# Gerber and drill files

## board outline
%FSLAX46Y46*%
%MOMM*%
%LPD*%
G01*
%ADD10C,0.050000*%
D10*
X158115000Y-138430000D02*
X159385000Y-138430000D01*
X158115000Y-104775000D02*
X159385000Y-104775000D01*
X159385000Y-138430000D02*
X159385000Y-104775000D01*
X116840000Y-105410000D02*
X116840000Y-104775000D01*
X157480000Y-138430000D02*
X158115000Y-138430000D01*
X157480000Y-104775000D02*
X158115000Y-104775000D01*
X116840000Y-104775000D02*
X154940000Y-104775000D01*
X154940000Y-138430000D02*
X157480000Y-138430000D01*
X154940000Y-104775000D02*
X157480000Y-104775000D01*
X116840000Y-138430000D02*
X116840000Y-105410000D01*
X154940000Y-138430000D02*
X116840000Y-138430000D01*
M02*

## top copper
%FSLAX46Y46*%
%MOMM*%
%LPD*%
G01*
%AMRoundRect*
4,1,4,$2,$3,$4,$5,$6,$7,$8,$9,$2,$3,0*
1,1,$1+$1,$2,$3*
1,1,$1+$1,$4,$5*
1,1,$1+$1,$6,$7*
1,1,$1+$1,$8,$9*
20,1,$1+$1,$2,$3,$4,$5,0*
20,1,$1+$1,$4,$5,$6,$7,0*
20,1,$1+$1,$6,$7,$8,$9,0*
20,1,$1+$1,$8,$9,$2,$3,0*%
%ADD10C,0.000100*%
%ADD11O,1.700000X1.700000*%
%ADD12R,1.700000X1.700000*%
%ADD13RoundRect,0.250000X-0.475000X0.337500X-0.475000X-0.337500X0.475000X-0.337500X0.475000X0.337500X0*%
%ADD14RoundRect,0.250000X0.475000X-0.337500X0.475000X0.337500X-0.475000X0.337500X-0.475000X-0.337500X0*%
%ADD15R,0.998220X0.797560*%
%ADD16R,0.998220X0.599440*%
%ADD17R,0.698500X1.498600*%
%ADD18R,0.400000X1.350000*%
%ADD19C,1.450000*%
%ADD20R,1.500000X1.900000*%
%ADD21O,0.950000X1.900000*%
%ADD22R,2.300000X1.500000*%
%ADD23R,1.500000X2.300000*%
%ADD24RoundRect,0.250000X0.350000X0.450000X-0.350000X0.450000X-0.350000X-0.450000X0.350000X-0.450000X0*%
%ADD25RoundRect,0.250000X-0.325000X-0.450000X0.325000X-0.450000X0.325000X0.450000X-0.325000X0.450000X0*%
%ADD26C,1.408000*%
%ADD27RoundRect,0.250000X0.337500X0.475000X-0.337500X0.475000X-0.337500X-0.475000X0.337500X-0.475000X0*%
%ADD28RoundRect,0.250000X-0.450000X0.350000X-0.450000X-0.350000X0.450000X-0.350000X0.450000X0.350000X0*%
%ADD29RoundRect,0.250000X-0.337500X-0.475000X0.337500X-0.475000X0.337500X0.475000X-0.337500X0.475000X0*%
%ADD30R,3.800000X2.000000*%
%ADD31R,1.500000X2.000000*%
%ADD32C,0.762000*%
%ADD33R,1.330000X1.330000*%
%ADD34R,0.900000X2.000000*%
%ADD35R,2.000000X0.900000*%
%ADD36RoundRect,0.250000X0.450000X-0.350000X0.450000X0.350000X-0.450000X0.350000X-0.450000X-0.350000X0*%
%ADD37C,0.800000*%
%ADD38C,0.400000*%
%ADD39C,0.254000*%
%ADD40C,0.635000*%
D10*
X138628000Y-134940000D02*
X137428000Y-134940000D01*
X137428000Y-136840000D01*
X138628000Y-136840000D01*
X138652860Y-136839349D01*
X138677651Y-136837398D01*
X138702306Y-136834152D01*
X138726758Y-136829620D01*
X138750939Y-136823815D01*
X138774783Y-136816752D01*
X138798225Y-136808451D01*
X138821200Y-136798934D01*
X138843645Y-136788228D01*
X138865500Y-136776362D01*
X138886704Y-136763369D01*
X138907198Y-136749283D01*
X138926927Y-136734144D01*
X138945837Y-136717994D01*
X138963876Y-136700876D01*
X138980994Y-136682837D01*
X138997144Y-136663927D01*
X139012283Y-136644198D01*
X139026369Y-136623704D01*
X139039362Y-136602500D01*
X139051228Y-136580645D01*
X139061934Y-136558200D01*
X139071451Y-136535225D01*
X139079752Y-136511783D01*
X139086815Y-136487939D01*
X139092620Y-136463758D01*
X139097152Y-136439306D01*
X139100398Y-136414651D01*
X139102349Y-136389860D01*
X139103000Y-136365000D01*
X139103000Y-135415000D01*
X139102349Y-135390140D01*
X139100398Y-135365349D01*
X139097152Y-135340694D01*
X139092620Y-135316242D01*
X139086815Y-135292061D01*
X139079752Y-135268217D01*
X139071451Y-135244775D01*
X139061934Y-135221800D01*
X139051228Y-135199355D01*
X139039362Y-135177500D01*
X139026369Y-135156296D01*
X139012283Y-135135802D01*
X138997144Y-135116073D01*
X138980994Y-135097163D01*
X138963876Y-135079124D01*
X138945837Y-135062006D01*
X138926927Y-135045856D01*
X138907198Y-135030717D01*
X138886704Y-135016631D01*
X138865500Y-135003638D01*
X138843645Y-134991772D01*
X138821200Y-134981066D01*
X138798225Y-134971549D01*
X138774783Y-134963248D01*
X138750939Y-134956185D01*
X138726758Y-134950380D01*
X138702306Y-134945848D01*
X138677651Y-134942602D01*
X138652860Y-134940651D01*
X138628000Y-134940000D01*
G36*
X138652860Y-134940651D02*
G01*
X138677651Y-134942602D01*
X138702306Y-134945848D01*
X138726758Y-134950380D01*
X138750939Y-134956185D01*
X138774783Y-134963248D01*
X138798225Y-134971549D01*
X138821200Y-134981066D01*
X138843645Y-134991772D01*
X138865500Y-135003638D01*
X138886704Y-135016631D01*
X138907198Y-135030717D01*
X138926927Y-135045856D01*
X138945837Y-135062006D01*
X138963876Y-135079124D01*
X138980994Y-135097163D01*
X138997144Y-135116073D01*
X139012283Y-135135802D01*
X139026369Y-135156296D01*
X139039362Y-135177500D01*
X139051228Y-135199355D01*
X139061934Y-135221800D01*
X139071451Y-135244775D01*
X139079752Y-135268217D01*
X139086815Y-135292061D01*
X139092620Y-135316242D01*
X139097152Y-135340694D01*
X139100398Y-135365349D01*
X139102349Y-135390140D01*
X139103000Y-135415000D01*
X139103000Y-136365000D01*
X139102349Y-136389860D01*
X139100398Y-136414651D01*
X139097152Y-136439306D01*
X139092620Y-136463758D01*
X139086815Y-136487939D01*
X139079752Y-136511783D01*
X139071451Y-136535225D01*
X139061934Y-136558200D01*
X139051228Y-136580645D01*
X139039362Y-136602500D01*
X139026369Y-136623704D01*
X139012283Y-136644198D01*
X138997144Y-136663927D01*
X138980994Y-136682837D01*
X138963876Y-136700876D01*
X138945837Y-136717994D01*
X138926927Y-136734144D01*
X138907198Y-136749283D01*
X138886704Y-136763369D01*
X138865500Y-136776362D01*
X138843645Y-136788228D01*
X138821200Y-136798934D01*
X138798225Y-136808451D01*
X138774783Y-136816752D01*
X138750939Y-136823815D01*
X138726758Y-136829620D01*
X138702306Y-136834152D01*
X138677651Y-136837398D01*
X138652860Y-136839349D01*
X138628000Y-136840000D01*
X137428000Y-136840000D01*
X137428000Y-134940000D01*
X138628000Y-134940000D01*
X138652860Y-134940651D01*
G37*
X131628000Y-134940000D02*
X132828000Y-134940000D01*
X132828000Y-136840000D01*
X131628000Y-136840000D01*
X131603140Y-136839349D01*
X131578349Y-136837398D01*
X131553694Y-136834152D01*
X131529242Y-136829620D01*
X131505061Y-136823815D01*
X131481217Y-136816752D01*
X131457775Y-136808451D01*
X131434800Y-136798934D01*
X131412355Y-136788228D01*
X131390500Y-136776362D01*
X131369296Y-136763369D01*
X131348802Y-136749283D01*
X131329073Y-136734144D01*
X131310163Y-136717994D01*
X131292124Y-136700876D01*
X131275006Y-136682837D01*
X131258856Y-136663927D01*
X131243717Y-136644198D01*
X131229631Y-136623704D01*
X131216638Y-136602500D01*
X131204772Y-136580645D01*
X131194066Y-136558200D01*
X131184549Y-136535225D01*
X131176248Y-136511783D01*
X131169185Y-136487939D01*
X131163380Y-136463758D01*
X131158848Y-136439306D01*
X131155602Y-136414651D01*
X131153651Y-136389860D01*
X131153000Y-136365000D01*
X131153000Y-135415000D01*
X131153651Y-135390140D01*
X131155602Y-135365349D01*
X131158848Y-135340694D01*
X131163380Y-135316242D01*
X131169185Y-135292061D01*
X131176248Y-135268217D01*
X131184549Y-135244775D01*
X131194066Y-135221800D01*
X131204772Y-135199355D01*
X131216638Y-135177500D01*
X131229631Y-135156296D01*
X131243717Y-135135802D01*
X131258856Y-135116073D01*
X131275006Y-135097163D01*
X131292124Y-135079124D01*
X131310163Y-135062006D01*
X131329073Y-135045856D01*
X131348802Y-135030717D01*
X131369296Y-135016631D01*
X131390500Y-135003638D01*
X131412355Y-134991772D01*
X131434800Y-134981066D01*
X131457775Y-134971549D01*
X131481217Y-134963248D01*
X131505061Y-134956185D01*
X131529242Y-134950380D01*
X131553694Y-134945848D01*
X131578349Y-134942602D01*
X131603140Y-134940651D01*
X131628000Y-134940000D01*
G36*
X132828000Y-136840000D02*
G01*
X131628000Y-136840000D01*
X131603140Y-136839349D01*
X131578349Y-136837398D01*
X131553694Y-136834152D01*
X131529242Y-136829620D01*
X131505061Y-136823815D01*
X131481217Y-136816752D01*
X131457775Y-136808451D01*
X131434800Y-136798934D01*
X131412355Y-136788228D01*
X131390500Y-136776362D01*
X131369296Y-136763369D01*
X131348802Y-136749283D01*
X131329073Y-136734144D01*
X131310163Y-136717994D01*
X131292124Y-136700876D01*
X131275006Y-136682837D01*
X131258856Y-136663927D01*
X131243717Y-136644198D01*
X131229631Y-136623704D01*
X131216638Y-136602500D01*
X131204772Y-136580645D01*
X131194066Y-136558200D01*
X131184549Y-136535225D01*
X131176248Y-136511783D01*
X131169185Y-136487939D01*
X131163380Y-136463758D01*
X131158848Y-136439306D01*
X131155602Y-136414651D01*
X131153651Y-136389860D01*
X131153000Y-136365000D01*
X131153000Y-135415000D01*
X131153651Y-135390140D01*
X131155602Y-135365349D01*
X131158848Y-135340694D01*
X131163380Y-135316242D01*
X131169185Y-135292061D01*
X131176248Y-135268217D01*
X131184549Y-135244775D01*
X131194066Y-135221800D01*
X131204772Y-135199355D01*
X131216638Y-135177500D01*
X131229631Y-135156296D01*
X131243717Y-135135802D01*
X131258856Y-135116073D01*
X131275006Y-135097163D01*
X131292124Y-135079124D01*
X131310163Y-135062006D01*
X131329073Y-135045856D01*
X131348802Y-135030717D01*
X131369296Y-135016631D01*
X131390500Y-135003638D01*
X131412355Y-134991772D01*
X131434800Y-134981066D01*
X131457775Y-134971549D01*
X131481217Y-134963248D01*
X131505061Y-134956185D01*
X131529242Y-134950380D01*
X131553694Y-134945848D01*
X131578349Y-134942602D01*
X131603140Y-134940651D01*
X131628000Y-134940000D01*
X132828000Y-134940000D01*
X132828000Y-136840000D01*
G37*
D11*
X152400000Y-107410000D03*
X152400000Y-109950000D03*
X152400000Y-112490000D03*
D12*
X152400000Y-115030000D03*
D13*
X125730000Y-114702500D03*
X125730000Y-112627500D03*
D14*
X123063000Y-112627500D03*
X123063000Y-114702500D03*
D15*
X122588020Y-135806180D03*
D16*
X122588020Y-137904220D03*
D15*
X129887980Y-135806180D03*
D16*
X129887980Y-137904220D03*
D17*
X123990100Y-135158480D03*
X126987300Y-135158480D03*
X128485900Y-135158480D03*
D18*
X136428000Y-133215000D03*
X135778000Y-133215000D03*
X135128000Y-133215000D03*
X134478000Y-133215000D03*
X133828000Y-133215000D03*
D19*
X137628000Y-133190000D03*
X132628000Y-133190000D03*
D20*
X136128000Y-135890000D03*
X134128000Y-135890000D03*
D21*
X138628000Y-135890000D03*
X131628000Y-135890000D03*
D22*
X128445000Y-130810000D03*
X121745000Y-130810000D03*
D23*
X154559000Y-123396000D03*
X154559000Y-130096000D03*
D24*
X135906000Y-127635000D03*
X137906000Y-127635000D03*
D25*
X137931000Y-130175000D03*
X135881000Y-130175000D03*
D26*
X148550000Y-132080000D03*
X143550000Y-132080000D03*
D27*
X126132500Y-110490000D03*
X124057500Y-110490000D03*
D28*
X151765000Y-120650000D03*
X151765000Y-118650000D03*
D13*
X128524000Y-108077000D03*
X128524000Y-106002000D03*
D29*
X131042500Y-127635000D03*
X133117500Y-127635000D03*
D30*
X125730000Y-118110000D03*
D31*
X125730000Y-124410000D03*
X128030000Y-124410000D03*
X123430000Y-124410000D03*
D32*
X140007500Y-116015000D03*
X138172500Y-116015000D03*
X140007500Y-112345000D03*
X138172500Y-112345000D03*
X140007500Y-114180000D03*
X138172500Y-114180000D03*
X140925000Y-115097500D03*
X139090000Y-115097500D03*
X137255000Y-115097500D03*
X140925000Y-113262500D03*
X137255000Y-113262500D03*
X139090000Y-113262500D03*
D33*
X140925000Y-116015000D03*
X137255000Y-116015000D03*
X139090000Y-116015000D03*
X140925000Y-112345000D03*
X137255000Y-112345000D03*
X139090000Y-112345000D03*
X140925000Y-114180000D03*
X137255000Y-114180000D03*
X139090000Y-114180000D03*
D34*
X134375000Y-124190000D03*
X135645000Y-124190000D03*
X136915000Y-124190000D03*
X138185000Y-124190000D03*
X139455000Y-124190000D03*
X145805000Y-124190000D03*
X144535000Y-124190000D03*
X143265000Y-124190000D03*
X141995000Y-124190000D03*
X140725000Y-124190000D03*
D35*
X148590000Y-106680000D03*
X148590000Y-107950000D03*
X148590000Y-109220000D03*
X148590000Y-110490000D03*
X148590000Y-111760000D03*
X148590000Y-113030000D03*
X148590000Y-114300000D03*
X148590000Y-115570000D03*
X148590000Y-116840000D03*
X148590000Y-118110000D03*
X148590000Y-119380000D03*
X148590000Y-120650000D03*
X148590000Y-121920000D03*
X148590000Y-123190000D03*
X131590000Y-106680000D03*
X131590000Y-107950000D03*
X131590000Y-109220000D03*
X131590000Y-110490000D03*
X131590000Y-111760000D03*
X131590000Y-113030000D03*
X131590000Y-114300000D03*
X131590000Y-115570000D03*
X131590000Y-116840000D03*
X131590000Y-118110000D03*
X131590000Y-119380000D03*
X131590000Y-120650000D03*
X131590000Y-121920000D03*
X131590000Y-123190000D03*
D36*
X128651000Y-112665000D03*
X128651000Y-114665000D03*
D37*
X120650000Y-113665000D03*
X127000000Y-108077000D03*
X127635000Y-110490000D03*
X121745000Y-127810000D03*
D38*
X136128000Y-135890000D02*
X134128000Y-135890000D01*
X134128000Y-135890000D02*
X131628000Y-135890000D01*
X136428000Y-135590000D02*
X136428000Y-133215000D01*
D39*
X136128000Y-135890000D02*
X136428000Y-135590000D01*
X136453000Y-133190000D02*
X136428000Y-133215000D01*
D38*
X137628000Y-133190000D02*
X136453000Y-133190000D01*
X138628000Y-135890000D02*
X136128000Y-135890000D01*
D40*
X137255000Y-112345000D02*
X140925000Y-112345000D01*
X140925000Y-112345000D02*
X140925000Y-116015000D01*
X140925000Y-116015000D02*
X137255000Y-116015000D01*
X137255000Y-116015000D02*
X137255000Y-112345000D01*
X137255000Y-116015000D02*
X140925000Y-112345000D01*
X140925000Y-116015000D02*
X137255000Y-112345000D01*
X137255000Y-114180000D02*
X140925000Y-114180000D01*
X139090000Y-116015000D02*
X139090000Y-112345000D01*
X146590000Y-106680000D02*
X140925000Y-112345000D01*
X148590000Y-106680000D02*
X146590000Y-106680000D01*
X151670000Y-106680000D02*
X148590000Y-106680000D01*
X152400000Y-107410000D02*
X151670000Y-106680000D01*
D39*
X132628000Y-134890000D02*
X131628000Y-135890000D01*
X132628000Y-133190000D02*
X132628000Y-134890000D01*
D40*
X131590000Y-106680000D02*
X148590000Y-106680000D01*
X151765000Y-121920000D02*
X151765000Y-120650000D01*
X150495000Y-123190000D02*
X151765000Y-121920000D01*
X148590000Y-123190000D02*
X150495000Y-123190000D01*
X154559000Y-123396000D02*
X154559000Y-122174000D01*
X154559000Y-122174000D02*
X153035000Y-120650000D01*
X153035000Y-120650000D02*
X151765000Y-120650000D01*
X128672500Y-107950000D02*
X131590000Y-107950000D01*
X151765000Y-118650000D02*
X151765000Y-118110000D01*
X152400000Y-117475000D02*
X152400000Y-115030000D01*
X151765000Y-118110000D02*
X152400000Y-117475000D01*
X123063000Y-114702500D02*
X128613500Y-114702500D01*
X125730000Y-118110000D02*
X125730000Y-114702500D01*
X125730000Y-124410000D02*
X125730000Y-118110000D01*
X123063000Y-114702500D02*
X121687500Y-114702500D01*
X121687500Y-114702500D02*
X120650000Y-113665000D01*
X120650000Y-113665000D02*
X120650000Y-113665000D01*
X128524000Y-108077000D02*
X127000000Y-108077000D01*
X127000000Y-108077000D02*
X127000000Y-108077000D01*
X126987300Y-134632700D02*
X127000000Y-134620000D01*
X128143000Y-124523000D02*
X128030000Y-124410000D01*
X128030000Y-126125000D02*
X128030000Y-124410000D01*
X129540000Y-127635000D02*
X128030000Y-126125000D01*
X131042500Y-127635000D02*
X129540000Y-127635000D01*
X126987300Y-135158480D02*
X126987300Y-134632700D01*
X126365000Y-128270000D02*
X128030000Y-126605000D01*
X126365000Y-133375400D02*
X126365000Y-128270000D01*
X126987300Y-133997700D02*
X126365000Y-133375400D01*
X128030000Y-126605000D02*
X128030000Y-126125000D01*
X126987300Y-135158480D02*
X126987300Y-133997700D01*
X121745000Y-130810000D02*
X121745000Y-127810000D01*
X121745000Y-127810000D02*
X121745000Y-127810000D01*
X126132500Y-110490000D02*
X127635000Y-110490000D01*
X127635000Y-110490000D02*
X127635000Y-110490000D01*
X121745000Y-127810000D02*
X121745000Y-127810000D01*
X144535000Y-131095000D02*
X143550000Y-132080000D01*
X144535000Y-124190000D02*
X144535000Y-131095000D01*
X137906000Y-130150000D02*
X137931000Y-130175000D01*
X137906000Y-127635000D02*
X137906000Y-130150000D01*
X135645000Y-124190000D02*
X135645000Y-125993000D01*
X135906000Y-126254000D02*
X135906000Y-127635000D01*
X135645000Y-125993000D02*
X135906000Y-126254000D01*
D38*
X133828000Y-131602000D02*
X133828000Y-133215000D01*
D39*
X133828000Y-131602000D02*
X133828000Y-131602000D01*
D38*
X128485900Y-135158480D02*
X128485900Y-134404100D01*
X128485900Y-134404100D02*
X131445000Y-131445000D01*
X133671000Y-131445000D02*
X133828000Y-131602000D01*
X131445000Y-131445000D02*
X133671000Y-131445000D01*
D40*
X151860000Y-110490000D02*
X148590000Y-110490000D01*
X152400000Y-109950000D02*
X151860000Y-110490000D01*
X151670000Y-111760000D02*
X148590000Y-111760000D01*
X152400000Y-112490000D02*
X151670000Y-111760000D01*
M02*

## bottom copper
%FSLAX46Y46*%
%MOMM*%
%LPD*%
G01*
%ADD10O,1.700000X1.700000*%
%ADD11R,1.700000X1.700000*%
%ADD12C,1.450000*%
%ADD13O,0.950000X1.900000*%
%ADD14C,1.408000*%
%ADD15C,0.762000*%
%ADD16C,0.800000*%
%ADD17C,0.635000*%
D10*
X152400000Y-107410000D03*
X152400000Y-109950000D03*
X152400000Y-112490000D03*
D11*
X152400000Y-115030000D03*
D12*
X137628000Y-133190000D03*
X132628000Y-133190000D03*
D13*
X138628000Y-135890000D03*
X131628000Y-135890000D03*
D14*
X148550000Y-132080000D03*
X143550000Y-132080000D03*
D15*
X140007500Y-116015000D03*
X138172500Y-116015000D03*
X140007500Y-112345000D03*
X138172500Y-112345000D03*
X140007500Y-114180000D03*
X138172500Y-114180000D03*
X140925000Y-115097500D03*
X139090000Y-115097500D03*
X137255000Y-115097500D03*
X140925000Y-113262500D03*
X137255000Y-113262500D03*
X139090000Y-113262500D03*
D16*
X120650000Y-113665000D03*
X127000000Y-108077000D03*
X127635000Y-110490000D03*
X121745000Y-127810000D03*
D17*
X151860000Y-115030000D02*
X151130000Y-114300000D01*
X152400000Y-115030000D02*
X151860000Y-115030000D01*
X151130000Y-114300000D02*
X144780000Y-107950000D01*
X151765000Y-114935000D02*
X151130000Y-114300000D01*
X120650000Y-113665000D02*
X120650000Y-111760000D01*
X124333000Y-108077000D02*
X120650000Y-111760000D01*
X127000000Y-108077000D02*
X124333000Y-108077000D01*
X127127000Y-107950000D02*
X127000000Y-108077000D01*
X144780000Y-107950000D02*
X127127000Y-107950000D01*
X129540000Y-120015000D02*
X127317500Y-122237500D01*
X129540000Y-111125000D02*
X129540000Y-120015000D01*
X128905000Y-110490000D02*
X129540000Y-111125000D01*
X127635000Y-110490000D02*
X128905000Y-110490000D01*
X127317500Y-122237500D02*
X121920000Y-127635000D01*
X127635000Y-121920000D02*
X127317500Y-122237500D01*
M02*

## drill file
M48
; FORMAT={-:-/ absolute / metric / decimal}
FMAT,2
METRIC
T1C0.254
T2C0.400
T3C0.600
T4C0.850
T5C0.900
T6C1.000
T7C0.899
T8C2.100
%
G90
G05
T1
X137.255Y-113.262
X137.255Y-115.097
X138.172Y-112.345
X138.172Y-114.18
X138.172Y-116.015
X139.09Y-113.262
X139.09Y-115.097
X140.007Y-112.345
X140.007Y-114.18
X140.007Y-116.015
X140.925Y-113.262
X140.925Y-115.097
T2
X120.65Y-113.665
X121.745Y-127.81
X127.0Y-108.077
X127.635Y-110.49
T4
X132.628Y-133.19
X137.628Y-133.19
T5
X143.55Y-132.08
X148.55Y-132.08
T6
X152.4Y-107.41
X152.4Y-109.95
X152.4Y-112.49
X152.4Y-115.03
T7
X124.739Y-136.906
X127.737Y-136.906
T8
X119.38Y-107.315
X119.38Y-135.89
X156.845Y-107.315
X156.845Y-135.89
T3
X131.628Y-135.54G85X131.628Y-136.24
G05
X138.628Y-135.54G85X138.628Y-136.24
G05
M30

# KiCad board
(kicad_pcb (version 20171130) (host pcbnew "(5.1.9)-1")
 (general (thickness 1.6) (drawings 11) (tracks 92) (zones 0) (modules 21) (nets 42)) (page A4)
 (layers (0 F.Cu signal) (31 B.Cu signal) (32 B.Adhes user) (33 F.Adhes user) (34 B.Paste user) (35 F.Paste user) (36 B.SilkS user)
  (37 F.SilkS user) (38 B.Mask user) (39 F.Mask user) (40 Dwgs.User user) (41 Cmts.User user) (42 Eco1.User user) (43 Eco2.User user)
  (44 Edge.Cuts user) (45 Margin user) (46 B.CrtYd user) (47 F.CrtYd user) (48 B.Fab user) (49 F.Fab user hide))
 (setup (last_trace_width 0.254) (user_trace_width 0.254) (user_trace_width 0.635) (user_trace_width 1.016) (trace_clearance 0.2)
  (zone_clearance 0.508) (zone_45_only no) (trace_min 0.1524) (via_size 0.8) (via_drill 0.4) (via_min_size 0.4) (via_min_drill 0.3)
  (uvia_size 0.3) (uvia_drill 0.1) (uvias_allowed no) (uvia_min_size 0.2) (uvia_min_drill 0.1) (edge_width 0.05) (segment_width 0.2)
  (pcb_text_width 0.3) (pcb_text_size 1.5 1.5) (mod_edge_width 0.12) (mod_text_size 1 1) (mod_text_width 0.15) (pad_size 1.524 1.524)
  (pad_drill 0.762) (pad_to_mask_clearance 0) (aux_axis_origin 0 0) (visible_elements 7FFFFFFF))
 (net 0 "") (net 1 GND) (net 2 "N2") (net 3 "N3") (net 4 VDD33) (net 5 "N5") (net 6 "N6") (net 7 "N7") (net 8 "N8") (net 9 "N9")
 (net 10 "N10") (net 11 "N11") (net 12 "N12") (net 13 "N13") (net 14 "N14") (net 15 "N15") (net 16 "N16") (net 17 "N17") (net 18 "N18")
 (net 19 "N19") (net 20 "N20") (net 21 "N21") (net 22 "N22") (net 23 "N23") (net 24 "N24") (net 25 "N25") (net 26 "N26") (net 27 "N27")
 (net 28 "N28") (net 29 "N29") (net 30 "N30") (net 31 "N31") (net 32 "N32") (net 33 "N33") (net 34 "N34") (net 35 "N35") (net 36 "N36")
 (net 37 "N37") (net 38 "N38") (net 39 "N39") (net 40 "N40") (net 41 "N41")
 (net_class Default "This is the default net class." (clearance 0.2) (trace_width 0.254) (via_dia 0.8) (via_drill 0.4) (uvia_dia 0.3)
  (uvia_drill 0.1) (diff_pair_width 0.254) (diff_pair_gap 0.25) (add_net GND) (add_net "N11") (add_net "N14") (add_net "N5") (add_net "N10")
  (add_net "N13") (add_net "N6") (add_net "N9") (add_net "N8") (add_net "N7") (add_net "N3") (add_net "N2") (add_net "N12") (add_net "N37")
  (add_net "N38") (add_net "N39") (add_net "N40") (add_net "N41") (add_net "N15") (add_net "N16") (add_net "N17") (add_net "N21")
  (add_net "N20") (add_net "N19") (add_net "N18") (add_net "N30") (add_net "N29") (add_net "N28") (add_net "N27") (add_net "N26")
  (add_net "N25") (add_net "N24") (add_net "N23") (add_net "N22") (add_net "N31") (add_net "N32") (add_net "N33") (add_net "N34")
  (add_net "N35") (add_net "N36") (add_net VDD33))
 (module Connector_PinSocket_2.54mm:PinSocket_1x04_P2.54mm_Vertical (layer F.Cu) (at 152.4 115.03 180)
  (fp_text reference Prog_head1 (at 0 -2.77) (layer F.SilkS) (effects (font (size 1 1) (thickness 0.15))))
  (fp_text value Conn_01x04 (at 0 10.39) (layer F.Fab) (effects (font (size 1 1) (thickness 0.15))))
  (pad 4 thru_hole oval (at 0 7.62 180) (size 1.7 1.7) (drill 1) (layers *.Cu *.Mask) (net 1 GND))
  (pad 3 thru_hole oval (at 0 5.08 180) (size 1.7 1.7) (drill 1) (layers *.Cu *.Mask) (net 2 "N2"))
  (pad 2 thru_hole oval (at 0 2.54 180) (size 1.7 1.7) (drill 1) (layers *.Cu *.Mask) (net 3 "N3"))
  (pad 1 thru_hole rect (at 0 0 180) (size 1.7 1.7) (drill 1) (layers *.Cu *.Mask) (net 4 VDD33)))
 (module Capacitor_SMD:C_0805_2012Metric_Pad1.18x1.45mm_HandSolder (layer F.Cu) (at 125.73 113.665 270)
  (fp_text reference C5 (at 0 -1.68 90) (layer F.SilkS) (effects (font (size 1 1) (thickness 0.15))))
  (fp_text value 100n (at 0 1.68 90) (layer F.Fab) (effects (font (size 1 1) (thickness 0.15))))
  (pad 2 smd roundrect (at 1.0375 0 270) (size 1.175 1.45) (layers F.Cu F.Paste F.Mask) (roundrect_rratio 0.212766) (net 4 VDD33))
  (pad 1 smd roundrect (at -1.0375 0 270) (size 1.175 1.45) (layers F.Cu F.Paste F.Mask) (roundrect_rratio 0.212766) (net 1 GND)))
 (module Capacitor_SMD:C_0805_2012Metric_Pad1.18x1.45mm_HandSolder (layer F.Cu) (at 123.063 113.665 90)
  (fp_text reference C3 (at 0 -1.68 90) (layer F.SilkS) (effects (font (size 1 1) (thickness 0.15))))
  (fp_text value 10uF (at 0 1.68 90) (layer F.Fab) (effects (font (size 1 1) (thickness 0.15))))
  (pad 2 smd roundrect (at 1.0375 0 90) (size 1.175 1.45) (layers F.Cu F.Paste F.Mask) (roundrect_rratio 0.212766) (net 1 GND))
  (pad 1 smd roundrect (at -1.0375 0 90) (size 1.175 1.45) (layers F.Cu F.Paste F.Mask) (roundrect_rratio 0.212766) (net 4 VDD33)))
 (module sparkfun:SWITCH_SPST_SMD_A (layer F.Cu) (at 126.238 136.906 180)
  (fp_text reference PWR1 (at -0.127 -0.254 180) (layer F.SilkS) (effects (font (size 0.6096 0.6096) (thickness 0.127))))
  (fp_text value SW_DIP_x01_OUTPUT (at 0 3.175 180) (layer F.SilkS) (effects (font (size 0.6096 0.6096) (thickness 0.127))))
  (pad "" np_thru_hole circle (at 1.4986 0 180) (size 0.89916 0.89916) (drill 0.89916) (layers *.Cu *.Mask) (solder_mask_margin 0.1016))
  (pad "" np_thru_hole circle (at -1.4986 0 180) (size 0.89916 0.89916) (drill 0.89916) (layers *.Cu *.Mask) (solder_mask_margin 0.1016))
  (pad GND4 smd rect (at 3.64998 1.09982 180) (size 0.99822 0.79756) (layers F.Cu F.Paste F.Mask) (solder_mask_margin 0.1016))
  (pad GND3 smd rect (at 3.64998 -0.99822 180) (size 0.99822 0.59944) (layers F.Cu F.Paste F.Mask) (solder_mask_margin 0.1016))
  (pad GND2 smd rect (at -3.64998 1.09982 180) (size 0.99822 0.79756) (layers F.Cu F.Paste F.Mask) (solder_mask_margin 0.1016))
  (pad GND1 smd rect (at -3.64998 -0.99822 180) (size 0.99822 0.59944) (layers F.Cu F.Paste F.Mask) (solder_mask_margin 0.1016))
  (pad 3 smd rect (at 2.2479 1.74752) (size 0.6985 1.4986) (layers F.Cu F.Paste F.Mask) (solder_mask_margin 0.1016))
  (pad 2 smd rect (at -0.7493 1.74752) (size 0.6985 1.4986) (layers F.Cu F.Paste F.Mask) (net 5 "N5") (solder_mask_margin 0.1016))
  (pad 1 smd rect (at -2.2479 1.74752) (size 0.6985 1.4986) (layers F.Cu F.Paste F.Mask) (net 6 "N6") (solder_mask_margin 0.1016)))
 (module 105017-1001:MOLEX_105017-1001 (layer F.Cu) (at 135.128 135.89)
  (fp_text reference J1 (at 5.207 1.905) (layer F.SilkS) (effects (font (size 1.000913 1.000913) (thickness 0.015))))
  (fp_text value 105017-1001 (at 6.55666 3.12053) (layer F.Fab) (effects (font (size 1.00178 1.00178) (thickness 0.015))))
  (fp_poly
   (pts (xy 3.5 -0.95) (xy 2.3 -0.95) (xy 2.3 0.95) (xy 3.5 0.95) (xy 3.52486 0.949349) (xy 3.549651 0.947398) (xy 3.574306 0.944152)
    (xy 3.598758 0.93962) (xy 3.622939 0.933815) (xy 3.646783 0.926752) (xy 3.670225 0.918451) (xy 3.6932 0.908934) (xy 3.715645 0.898228)
    (xy 3.7375 0.886362) (xy 3.758704 0.873369) (xy 3.779198 0.859283) (xy 3.798927 0.844144) (xy 3.817837 0.827994) (xy 3.835876 0.810876)
    (xy 3.852994 0.792837) (xy 3.869144 0.773927) (xy 3.884283 0.754198) (xy 3.898369 0.733704) (xy 3.911362 0.7125) (xy 3.923228 0.690645)
    (xy 3.933934 0.6682) (xy 3.943451 0.645225) (xy 3.951752 0.621783) (xy 3.958815 0.597939) (xy 3.96462 0.573758) (xy 3.969152 0.549306)
    (xy 3.972398 0.524651) (xy 3.974349 0.49986) (xy 3.975 0.475) (xy 3.975 -0.475) (xy 3.974349 -0.49986) (xy 3.972398 -0.524651)
    (xy 3.969152 -0.549306) (xy 3.96462 -0.573758) (xy 3.958815 -0.597939) (xy 3.951752 -0.621783) (xy 3.943451 -0.645225)
    (xy 3.933934 -0.6682) (xy 3.923228 -0.690645) (xy 3.911362 -0.7125) (xy 3.898369 -0.733704) (xy 3.884283 -0.754198)
    (xy 3.869144 -0.773927) (xy 3.852994 -0.792837) (xy 3.835876 -0.810876) (xy 3.817837 -0.827994) (xy 3.798927 -0.844144)
    (xy 3.779198 -0.859283) (xy 3.758704 -0.873369) (xy 3.7375 -0.886362) (xy 3.715645 -0.898228) (xy 3.6932 -0.908934)
    (xy 3.670225 -0.918451) (xy 3.646783 -0.926752) (xy 3.622939 -0.933815) (xy 3.598758 -0.93962) (xy 3.574306 -0.944152)
    (xy 3.549651 -0.947398) (xy 3.52486 -0.949349) (xy 3.5 -0.95))
   (layer F.Cu) (width 0.0001))
  (fp_poly
   (pts (xy -3.5 -0.95) (xy -2.3 -0.95) (xy -2.3 0.95) (xy -3.5 0.95) (xy -3.52486 0.949349) (xy -3.549651 0.947398) (xy -3.574306 0.944152)
    (xy -3.598758 0.93962) (xy -3.622939 0.933815) (xy -3.646783 0.926752) (xy -3.670225 0.918451) (xy -3.6932 0.908934)
    (xy -3.715645 0.898228) (xy -3.7375 0.886362) (xy -3.758704 0.873369) (xy -3.779198 0.859283) (xy -3.798927 0.844144)
    (xy -3.817837 0.827994) (xy -3.835876 0.810876) (xy -3.852994 0.792837) (xy -3.869144 0.773927) (xy -3.884283 0.754198)
    (xy -3.898369 0.733704) (xy -3.911362 0.7125) (xy -3.923228 0.690645) (xy -3.933934 0.6682) (xy -3.943451 0.645225)
    (xy -3.951752 0.621783) (xy -3.958815 0.597939) (xy -3.96462 0.573758) (xy -3.969152 0.549306) (xy -3.972398 0.524651)
    (xy -3.974349 0.49986) (xy -3.975 0.475) (xy -3.975 -0.475) (xy -3.974349 -0.49986) (xy -3.972398 -0.524651) (xy -3.969152 -0.549306)
    (xy -3.96462 -0.573758) (xy -3.958815 -0.597939) (xy -3.951752 -0.621783) (xy -3.943451 -0.645225) (xy -3.933934 -0.6682)
    (xy -3.923228 -0.690645) (xy -3.911362 -0.7125) (xy -3.898369 -0.733704) (xy -3.884283 -0.754198) (xy -3.869144 -0.773927)
    (xy -3.852994 -0.792837) (xy -3.835876 -0.810876) (xy -3.817837 -0.827994) (xy -3.798927 -0.844144) (xy -3.779198 -0.859283)
    (xy -3.758704 -0.873369) (xy -3.7375 -0.886362) (xy -3.715645 -0.898228) (xy -3.6932 -0.908934) (xy -3.670225 -0.918451)
    (xy -3.646783 -0.926752) (xy -3.622939 -0.933815) (xy -3.598758 -0.93962) (xy -3.574306 -0.944152) (xy -3.549651 -0.947398)
    (xy -3.52486 -0.949349) (xy -3.5 -0.95))
   (layer F.Cu) (width 0.0001))
  (pad 5 smd rect (at 1.3 -2.675) (size 0.4 1.35) (layers F.Cu F.Paste F.Mask) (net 1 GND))
  (pad 4 smd rect (at 0.65 -2.675) (size 0.4 1.35) (layers F.Cu F.Paste F.Mask) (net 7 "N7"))
  (pad 3 smd rect (at 0 -2.675) (size 0.4 1.35) (layers F.Cu F.Paste F.Mask) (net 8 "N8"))
  (pad 2 smd rect (at -0.65 -2.675) (size 0.4 1.35) (layers F.Cu F.Paste F.Mask) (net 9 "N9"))
  (pad 1 smd rect (at -1.3 -2.675) (size 0.4 1.35) (layers F.Cu F.Paste F.Mask) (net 6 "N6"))
  (pad S4 thru_hole circle (at 2.5 -2.7) (size 1.45 1.45) (drill 0.85) (layers *.Cu *.Mask) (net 1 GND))
  (pad S3 thru_hole circle (at -2.5 -2.7) (size 1.45 1.45) (drill 0.85) (layers *.Cu *.Mask) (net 1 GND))
  (pad S6 smd rect (at 1 0) (size 1.5 1.9) (layers F.Cu F.Paste F.Mask) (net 1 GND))
  (pad S5 smd rect (at -1 0) (size 1.5 1.9) (layers F.Cu F.Paste F.Mask) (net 1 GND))
  (pad S2 thru_hole oval (at 3.5 0) (size 0.95 1.9) (drill oval 0.6 1.3) (layers *.Cu) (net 1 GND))
  (pad S1 thru_hole oval (at -3.5 0) (size 0.95 1.9) (drill oval 0.6 1.3) (layers *.Cu) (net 1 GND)))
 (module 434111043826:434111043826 (layer F.Cu) (at 125.095 130.81)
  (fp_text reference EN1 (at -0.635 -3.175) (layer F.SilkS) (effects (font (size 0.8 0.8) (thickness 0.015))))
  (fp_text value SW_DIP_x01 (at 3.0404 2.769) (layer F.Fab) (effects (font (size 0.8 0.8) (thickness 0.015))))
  (pad 2 smd rect (at 3.35 0) (size 2.3 1.5) (layers F.Cu F.Paste F.Mask) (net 1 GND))
  (pad 1 smd rect (at -3.35 0) (size 2.3 1.5) (layers F.Cu F.Paste F.Mask) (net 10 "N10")))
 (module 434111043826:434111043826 (layer F.Cu) (at 154.559 126.746 270)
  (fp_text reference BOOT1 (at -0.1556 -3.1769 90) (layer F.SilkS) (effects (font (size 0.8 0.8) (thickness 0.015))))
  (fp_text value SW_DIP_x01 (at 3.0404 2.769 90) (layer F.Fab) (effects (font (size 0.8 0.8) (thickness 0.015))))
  (pad 1 smd rect (at -3.35 0 270) (size 2.3 1.5) (layers F.Cu F.Paste F.Mask) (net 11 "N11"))
  (pad 2 smd rect (at 3.35 0 270) (size 2.3 1.5) (layers F.Cu F.Paste F.Mask) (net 1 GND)))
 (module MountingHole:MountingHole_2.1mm (layer F.Cu) (at 156.845 135.89)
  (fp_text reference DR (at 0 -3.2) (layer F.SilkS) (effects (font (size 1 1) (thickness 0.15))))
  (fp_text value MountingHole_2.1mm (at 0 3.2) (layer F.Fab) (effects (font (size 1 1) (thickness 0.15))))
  (pad "" np_thru_hole circle (at 0 0) (size 2.1 2.1) (drill 2.1) (layers *.Cu *.Mask)))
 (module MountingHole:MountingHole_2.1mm (layer F.Cu) (at 119.38 107.315)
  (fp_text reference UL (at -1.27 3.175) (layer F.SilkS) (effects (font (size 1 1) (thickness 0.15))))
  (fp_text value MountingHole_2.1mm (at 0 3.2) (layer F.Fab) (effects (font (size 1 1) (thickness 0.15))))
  (pad "" np_thru_hole circle (at 0 0) (size 2.1 2.1) (drill 2.1) (layers *.Cu *.Mask)))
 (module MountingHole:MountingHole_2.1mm (layer F.Cu) (at 156.845 107.315)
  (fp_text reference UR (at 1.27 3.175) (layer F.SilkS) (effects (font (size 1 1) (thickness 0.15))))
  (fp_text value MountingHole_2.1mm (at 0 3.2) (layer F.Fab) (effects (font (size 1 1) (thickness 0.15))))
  (pad "" np_thru_hole circle (at 0 0) (size 2.1 2.1) (drill 2.1) (layers *.Cu *.Mask)))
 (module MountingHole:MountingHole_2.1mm (layer F.Cu) (at 119.38 135.89)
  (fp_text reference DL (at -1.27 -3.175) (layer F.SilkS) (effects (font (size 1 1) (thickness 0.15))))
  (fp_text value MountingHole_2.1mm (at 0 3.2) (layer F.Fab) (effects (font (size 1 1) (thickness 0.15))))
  (pad "" np_thru_hole circle (at 0 0) (size 2.1 2.1) (drill 2.1) (layers *.Cu *.Mask)))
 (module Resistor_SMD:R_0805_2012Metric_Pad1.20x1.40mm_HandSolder (layer F.Cu) (at 136.906 127.635 180)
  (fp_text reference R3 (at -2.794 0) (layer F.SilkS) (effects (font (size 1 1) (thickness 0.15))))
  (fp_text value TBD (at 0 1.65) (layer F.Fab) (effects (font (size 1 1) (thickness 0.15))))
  (pad 2 smd roundrect (at 1 0 180) (size 1.2 1.4) (layers F.Cu F.Paste F.Mask) (roundrect_rratio 0.208333) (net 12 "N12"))
  (pad 1 smd roundrect (at -1 0 180) (size 1.2 1.4) (layers F.Cu F.Paste F.Mask) (roundrect_rratio 0.208333) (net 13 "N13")))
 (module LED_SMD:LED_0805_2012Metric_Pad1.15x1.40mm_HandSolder (layer F.Cu) (at 136.906 130.175)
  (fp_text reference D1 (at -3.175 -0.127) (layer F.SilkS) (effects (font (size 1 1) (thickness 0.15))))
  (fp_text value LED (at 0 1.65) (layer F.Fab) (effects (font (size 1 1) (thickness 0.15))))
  (pad 2 smd roundrect (at 1.025 0) (size 1.15 1.4) (layers F.Cu F.Paste F.Mask) (roundrect_rratio 0.217391) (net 13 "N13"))
  (pad 1 smd roundrect (at -1.025 0) (size 1.15 1.4) (layers F.Cu F.Paste F.Mask) (roundrect_rratio 0.217391) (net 1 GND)))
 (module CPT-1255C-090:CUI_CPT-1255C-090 (layer F.Cu) (at 146.05 132.08)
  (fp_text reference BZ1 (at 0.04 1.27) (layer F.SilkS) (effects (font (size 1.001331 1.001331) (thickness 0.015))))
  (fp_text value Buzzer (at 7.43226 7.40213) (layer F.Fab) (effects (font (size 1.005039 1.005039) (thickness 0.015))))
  (pad 2 thru_hole circle (at 2.5 0) (size 1.408 1.408) (drill 0.9) (layers *.Cu *.Mask) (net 1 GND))
  (pad 1 thru_hole circle (at -2.5 0) (size 1.408 1.408) (drill 0.9) (layers *.Cu *.Mask) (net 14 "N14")))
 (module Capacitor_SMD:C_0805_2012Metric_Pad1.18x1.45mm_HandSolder (layer F.Cu) (at 125.095 110.49 180)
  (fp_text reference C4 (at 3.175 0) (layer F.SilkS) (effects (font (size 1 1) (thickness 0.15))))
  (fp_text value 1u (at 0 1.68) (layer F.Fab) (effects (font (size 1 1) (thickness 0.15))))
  (pad 1 smd roundrect (at -1.0375 0 180) (size 1.175 1.45) (layers F.Cu F.Paste F.Mask) (roundrect_rratio 0.212766) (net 10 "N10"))
  (pad 2 smd roundrect (at 1.0375 0 180) (size 1.175 1.45) (layers F.Cu F.Paste F.Mask) (roundrect_rratio 0.212766) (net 1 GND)))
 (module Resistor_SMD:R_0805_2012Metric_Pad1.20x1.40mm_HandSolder (layer F.Cu) (at 151.765 119.65 270)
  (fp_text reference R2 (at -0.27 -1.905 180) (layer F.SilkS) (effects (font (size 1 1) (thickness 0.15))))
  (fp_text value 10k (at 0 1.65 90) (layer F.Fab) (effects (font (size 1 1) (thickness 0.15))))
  (pad 2 smd roundrect (at 1 0 270) (size 1.2 1.4) (layers F.Cu F.Paste F.Mask) (roundrect_rratio 0.208333) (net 11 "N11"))
  (pad 1 smd roundrect (at -1 0 270) (size 1.2 1.4) (layers F.Cu F.Paste F.Mask) (roundrect_rratio 0.208333) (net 4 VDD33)))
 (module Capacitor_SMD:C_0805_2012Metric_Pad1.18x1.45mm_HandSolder (layer F.Cu) (at 128.524 107.0395 270)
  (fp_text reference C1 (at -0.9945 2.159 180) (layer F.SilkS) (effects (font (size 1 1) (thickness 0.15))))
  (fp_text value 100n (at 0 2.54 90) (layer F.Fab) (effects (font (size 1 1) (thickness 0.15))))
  (pad 2 smd roundrect (at 1.0375 0 270) (size 1.175 1.45) (layers F.Cu F.Paste F.Mask) (roundrect_rratio 0.212766) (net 4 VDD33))
  (pad 1 smd roundrect (at -1.0375 0 270) (size 1.175 1.45) (layers F.Cu F.Paste F.Mask) (roundrect_rratio 0.212766) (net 1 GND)))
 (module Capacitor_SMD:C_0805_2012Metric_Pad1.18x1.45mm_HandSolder (layer F.Cu) (at 132.08 127.635)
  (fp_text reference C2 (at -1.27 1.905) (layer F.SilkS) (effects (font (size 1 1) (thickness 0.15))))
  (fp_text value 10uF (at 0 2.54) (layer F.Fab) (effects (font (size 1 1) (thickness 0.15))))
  (pad 1 smd roundrect (at -1.0375 0) (size 1.175 1.45) (layers F.Cu F.Paste F.Mask) (roundrect_rratio 0.212766) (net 5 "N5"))
  (pad 2 smd roundrect (at 1.0375 0) (size 1.175 1.45) (layers F.Cu F.Paste F.Mask) (roundrect_rratio 0.212766) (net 1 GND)))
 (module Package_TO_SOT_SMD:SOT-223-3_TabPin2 (layer F.Cu) (at 125.73 121.26 90)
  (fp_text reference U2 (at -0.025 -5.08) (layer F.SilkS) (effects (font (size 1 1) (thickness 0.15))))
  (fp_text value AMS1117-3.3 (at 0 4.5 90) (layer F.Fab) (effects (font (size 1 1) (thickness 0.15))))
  (pad 2 smd rect (at 3.15 0 90) (size 2 3.8) (layers F.Cu F.Paste F.Mask) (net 4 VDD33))
  (pad 2 smd rect (at -3.15 0 90) (size 2 1.5) (layers F.Cu F.Paste F.Mask) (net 4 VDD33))
  (pad 3 smd rect (at -3.15 2.3 90) (size 2 1.5) (layers F.Cu F.Paste F.Mask) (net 5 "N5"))
  (pad 1 smd rect (at -3.15 -2.3 90) (size 2 1.5) (layers F.Cu F.Paste F.Mask) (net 1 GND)))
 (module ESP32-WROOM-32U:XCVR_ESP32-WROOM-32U (layer F.Cu) (at 140.09 115.09)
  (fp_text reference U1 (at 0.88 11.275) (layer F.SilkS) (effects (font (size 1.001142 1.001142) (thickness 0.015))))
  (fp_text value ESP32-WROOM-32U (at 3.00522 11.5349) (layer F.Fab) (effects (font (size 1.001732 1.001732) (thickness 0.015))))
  (pad G.21 thru_hole circle (at -0.0825 0.925) (size 0.762 0.762) (drill 0.254) (layers *.Cu *.Mask) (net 1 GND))
  (pad G.22 thru_hole circle (at -1.9175 0.925) (size 0.762 0.762) (drill 0.254) (layers *.Cu *.Mask) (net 1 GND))
  (pad G.11 thru_hole circle (at -0.0825 -2.745) (size 0.762 0.762) (drill 0.254) (layers *.Cu *.Mask) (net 1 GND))
  (pad G.12 thru_hole circle (at -1.9175 -2.745) (size 0.762 0.762) (drill 0.254) (layers *.Cu *.Mask) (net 1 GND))
  (pad G.16 thru_hole circle (at -0.0825 -0.91) (size 0.762 0.762) (drill 0.254) (layers *.Cu *.Mask) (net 1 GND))
  (pad G.17 thru_hole circle (at -1.9175 -0.91) (size 0.762 0.762) (drill 0.254) (layers *.Cu *.Mask) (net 1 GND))
  (pad G.18 thru_hole circle (at 0.835 0.0075) (size 0.762 0.762) (drill 0.254) (layers *.Cu *.Mask) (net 1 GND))
  (pad G.19 thru_hole circle (at -1 0.0075) (size 0.762 0.762) (drill 0.254) (layers *.Cu *.Mask) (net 1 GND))
  (pad G.20 thru_hole circle (at -2.835 0.0075) (size 0.762 0.762) (drill 0.254) (layers *.Cu *.Mask) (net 1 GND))
  (pad G.13 thru_hole circle (at 0.835 -1.8275) (size 0.762 0.762) (drill 0.254) (layers *.Cu *.Mask) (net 1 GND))
  (pad G.15 thru_hole circle (at -2.835 -1.8275) (size 0.762 0.762) (drill 0.254) (layers *.Cu *.Mask) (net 1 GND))
  (pad G.14 thru_hole circle (at -1 -1.8275) (size 0.762 0.762) (drill 0.254) (layers *.Cu *.Mask) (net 1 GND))
  (pad G.8 smd rect (at 0.835 0.925) (size 1.33 1.33) (layers F.Cu F.Paste F.Mask) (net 1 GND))
  (pad G.10 smd rect (at -2.835 0.925) (size 1.33 1.33) (layers F.Cu F.Paste F.Mask) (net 1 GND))
  (pad G.9 smd rect (at -1 0.925) (size 1.33 1.33) (layers F.Cu F.Paste F.Mask) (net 1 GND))
  (pad G.1 smd rect (at 0.835 -2.745) (size 1.33 1.33) (layers F.Cu F.Paste F.Mask) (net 1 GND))
  (pad G.4 smd rect (at -2.835 -2.745) (size 1.33 1.33) (layers F.Cu F.Paste F.Mask) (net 1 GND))
  (pad G.2 smd rect (at -1 -2.745) (size 1.33 1.33) (layers F.Cu F.Paste F.Mask) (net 1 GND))
  (pad G.5 smd rect (at 0.835 -0.91) (size 1.33 1.33) (layers F.Cu F.Paste F.Mask) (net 1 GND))
  (pad G.7 smd rect (at -2.835 -0.91) (size 1.33 1.33) (layers F.Cu F.Paste F.Mask) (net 1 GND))
  (pad G.6 smd rect (at -1 -0.91) (size 1.33 1.33) (layers F.Cu F.Paste F.Mask) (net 1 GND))
  (pad 15 smd rect (at -5.715 9.1) (size 0.9 2) (layers F.Cu F.Paste F.Mask) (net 1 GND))
  (pad 16 smd rect (at -4.445 9.1) (size 0.9 2) (layers F.Cu F.Paste F.Mask) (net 12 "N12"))
  (pad 17 smd rect (at -3.175 9.1) (size 0.9 2) (layers F.Cu F.Paste F.Mask) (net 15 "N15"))
  (pad 18 smd rect (at -1.905 9.1) (size 0.9 2) (layers F.Cu F.Paste F.Mask) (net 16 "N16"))
  (pad 19 smd rect (at -0.635 9.1) (size 0.9 2) (layers F.Cu F.Paste F.Mask) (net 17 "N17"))
  (pad 24 smd rect (at 5.715 9.1) (size 0.9 2) (layers F.Cu F.Paste F.Mask) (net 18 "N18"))
  (pad 23 smd rect (at 4.445 9.1) (size 0.9 2) (layers F.Cu F.Paste F.Mask) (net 14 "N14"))
  (pad 22 smd rect (at 3.175 9.1) (size 0.9 2) (layers F.Cu F.Paste F.Mask) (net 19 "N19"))
  (pad 21 smd rect (at 1.905 9.1) (size 0.9 2) (layers F.Cu F.Paste F.Mask) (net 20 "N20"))
  (pad 20 smd rect (at 0.635 9.1) (size 0.9 2) (layers F.Cu F.Paste F.Mask) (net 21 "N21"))
  (pad 38 smd rect (at 8.5 -8.41) (size 2 0.9) (layers F.Cu F.Paste F.Mask) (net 1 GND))
  (pad 37 smd rect (at 8.5 -7.14) (size 2 0.9) (layers F.Cu F.Paste F.Mask) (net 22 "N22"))
  (pad 36 smd rect (at 8.5 -5.87) (size 2 0.9) (layers F.Cu F.Paste F.Mask) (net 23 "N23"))
  (pad 35 smd rect (at 8.5 -4.6) (size 2 0.9) (layers F.Cu F.Paste F.Mask) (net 2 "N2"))
  (pad 34 smd rect (at 8.5 -3.33) (size 2 0.9) (layers F.Cu F.Paste F.Mask) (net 3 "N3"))
  (pad 33 smd rect (at 8.5 -2.06) (size 2 0.9) (layers F.Cu F.Paste F.Mask) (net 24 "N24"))
  (pad 32 smd rect (at 8.5 -0.79) (size 2 0.9) (layers F.Cu F.Paste F.Mask))
  (pad 31 smd rect (at 8.5 0.48) (size 2 0.9) (layers F.Cu F.Paste F.Mask) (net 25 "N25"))
  (pad 30 smd rect (at 8.5 1.75) (size 2 0.9) (layers F.Cu F.Paste F.Mask) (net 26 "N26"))
  (pad 29 smd rect (at 8.5 3.02) (size 2 0.9) (layers F.Cu F.Paste F.Mask) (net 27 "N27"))
  (pad 28 smd rect (at 8.5 4.29) (size 2 0.9) (layers F.Cu F.Paste F.Mask) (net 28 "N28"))
  (pad 27 smd rect (at 8.5 5.56) (size 2 0.9) (layers F.Cu F.Paste F.Mask) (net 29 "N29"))
  (pad 26 smd rect (at 8.5 6.83) (size 2 0.9) (layers F.Cu F.Paste F.Mask) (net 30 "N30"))
  (pad 25 smd rect (at 8.5 8.1) (size 2 0.9) (layers F.Cu F.Paste F.Mask) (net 11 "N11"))
  (pad 1 smd rect (at -8.5 -8.41) (size 2 0.9) (layers F.Cu F.Paste F.Mask) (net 1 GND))
  (pad 2 smd rect (at -8.5 -7.14) (size 2 0.9) (layers F.Cu F.Paste F.Mask) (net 4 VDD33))
  (pad 3 smd rect (at -8.5 -5.87) (size 2 0.9) (layers F.Cu F.Paste F.Mask) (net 10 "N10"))
  (pad 4 smd rect (at -8.5 -4.6) (size 2 0.9) (layers F.Cu F.Paste F.Mask) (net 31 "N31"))
  (pad 5 smd rect (at -8.5 -3.33) (size 2 0.9) (layers F.Cu F.Paste F.Mask) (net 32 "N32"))
  (pad 6 smd rect (at -8.5 -2.06) (size 2 0.9) (layers F.Cu F.Paste F.Mask) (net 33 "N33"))
  (pad 7 smd rect (at -8.5 -0.79) (size 2 0.9) (layers F.Cu F.Paste F.Mask) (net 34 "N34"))
  (pad 8 smd rect (at -8.5 0.48) (size 2 0.9) (layers F.Cu F.Paste F.Mask) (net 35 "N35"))
  (pad 9 smd rect (at -8.5 1.75) (size 2 0.9) (layers F.Cu F.Paste F.Mask) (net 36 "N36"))
  (pad 10 smd rect (at -8.5 3.02) (size 2 0.9) (layers F.Cu F.Paste F.Mask) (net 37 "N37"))
  (pad 11 smd rect (at -8.5 4.29) (size 2 0.9) (layers F.Cu F.Paste F.Mask) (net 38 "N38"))
  (pad 12 smd rect (at -8.5 5.56) (size 2 0.9) (layers F.Cu F.Paste F.Mask) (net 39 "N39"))
  (pad 13 smd rect (at -8.5 6.83) (size 2 0.9) (layers F.Cu F.Paste F.Mask) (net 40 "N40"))
  (pad 14 smd rect (at -8.5 8.1) (size 2 0.9) (layers F.Cu F.Paste F.Mask) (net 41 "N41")))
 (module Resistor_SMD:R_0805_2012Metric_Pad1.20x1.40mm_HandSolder (layer F.Cu) (at 128.651 113.665 90)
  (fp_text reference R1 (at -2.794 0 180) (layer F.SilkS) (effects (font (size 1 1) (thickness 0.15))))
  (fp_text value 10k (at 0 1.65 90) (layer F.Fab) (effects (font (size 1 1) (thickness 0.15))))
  (pad 2 smd roundrect (at 1 0 90) (size 1.2 1.4) (layers F.Cu F.Paste F.Mask) (roundrect_rratio 0.208333) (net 10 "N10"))
  (pad 1 smd roundrect (at -1 0 90) (size 1.2 1.4) (layers F.Cu F.Paste F.Mask) (roundrect_rratio 0.208333) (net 4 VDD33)))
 (gr_line (start 158.115 138.43) (end 159.385 138.43) (layer Edge.Cuts) (width 0.05))
 (gr_line (start 158.115 104.775) (end 159.385 104.775) (layer Edge.Cuts) (width 0.05))
 (gr_line (start 159.385 138.43) (end 159.385 104.775) (layer Edge.Cuts) (width 0.05))
 (gr_line (start 116.84 105.41) (end 116.84 104.775) (layer Edge.Cuts) (width 0.05))
 (gr_line (start 157.48 138.43) (end 158.115 138.43) (layer Edge.Cuts) (width 0.05))
 (gr_line (start 157.48 104.775) (end 158.115 104.775) (layer Edge.Cuts) (width 0.05))
 (gr_line (start 116.84 104.775) (end 154.94 104.775) (layer Edge.Cuts) (width 0.05))
 (gr_line (start 154.94 138.43) (end 157.48 138.43) (layer Edge.Cuts) (width 0.05))
 (gr_line (start 154.94 104.775) (end 157.48 104.775) (layer Edge.Cuts) (width 0.05))
 (gr_line (start 116.84 138.43) (end 116.84 105.41) (layer Edge.Cuts) (width 0.05))
 (gr_line (start 154.94 138.43) (end 116.84 138.43) (layer Edge.Cuts) (width 0.05))
 (segment (start 136.128 135.89) (end 134.128 135.89) (width 0.4) (layer F.Cu) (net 1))
 (segment (start 134.128 135.89) (end 131.628 135.89) (width 0.4) (layer F.Cu) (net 1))
 (segment (start 136.428 135.59) (end 136.428 133.215) (width 0.4) (layer F.Cu) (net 1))
 (segment (start 136.128 135.89) (end 136.428 135.59) (width 0.254) (layer F.Cu) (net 1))
 (segment (start 136.453 133.19) (end 136.428 133.215) (width 0.254) (layer F.Cu) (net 1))
 (segment (start 137.628 133.19) (end 136.453 133.19) (width 0.4) (layer F.Cu) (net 1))
 (segment (start 138.628 135.89) (end 136.128 135.89) (width 0.4) (layer F.Cu) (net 1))
 (segment (start 137.255 112.345) (end 140.925 112.345) (width 0.635) (layer F.Cu) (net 1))
 (segment (start 140.925 112.345) (end 140.925 116.015) (width 0.635) (layer F.Cu) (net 1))
 (segment (start 140.925 116.015) (end 137.255 116.015) (width 0.635) (layer F.Cu) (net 1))
 (segment (start 137.255 116.015) (end 137.255 112.345) (width 0.635) (layer F.Cu) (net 1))
 (segment (start 137.255 116.015) (end 140.925 112.345) (width 0.635) (layer F.Cu) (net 1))
 (segment (start 140.925 116.015) (end 137.255 112.345) (width 0.635) (layer F.Cu) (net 1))
 (segment (start 137.255 114.18) (end 140.925 114.18) (width 0.635) (layer F.Cu) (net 1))
 (segment (start 139.09 116.015) (end 139.09 112.345) (width 0.635) (layer F.Cu) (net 1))
 (segment (start 146.59 106.68) (end 140.925 112.345) (width 0.635) (layer F.Cu) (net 1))
 (segment (start 148.59 106.68) (end 146.59 106.68) (width 0.635) (layer F.Cu) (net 1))
 (segment (start 151.67 106.68) (end 148.59 106.68) (width 0.635) (layer F.Cu) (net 1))
 (segment (start 152.4 107.41) (end 151.67 106.68) (width 0.635) (layer F.Cu) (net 1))
 (segment (start 132.628 134.89) (end 131.628 135.89) (width 0.254) (layer F.Cu) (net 1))
 (segment (start 132.628 133.19) (end 132.628 134.89) (width 0.254) (layer F.Cu) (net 1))
 (segment (start 131.59 106.68) (end 148.59 106.68) (width 0.635) (layer F.Cu) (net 1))
 (segment (start 151.765 121.92) (end 151.765 120.65) (width 0.635) (layer F.Cu) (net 11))
 (segment (start 150.495 123.19) (end 151.765 121.92) (width 0.635) (layer F.Cu) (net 11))
 (segment (start 148.59 123.19) (end 150.495 123.19) (width 0.635) (layer F.Cu) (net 11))
 (segment (start 154.559 123.396) (end 154.559 122.174) (width 0.635) (layer F.Cu) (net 11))
 (segment (start 154.559 122.174) (end 153.035 120.65) (width 0.635) (layer F.Cu) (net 11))
 (segment (start 153.035 120.65) (end 151.765 120.65) (width 0.635) (layer F.Cu) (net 11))
 (segment (start 151.86 115.03) (end 151.13 114.3) (width 0.635) (layer B.Cu) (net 4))
 (segment (start 152.4 115.03) (end 151.86 115.03) (width 0.635) (layer B.Cu) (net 4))
 (segment (start 151.13 114.3) (end 144.78 107.95) (width 0.635) (layer B.Cu) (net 4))
 (segment (start 151.765 114.935) (end 151.13 114.3) (width 0.635) (layer B.Cu) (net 4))
 (segment (start 128.6725 107.95) (end 131.59 107.95) (width 0.635) (layer F.Cu) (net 4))
 (segment (start 151.765 118.65) (end 151.765 118.11) (width 0.635) (layer F.Cu) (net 4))
 (segment (start 152.4 117.475) (end 152.4 115.03) (width 0.635) (layer F.Cu) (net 4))
 (segment (start 151.765 118.11) (end 152.4 117.475) (width 0.635) (layer F.Cu) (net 4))
 (segment (start 123.063 114.7025) (end 128.6135 114.7025) (width 0.635) (layer F.Cu) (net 4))
 (segment (start 125.73 118.11) (end 125.73 114.7025) (width 0.635) (layer F.Cu) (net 4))
 (segment (start 125.73 124.41) (end 125.73 118.11) (width 0.635) (layer F.Cu) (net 4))
 (segment (start 123.063 114.7025) (end 121.6875 114.7025) (width 0.635) (layer F.Cu) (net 4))
 (segment (start 121.6875 114.7025) (end 120.65 113.665) (width 0.635) (layer F.Cu) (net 4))
 (segment (start 120.65 113.665) (end 120.65 113.665) (width 0.635) (layer F.Cu) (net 4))
 (via (at 120.65 113.665) (size 0.8) (drill 0.4) (layers F.Cu B.Cu) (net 4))
 (segment (start 120.65 113.665) (end 120.65 111.76) (width 0.635) (layer B.Cu) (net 4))
 (segment (start 128.524 108.077) (end 127 108.077) (width 0.635) (layer F.Cu) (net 4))
 (segment (start 127 108.077) (end 127 108.077) (width 0.635) (layer F.Cu) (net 4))
 (via (at 127 108.077) (size 0.8) (drill 0.4) (layers F.Cu B.Cu) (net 4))
 (segment (start 124.333 108.077) (end 120.65 111.76) (width 0.635) (layer B.Cu) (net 4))
 (segment (start 127 108.077) (end 124.333 108.077) (width 0.635) (layer B.Cu) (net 4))
 (segment (start 127.127 107.95) (end 127 108.077) (width 0.635) (layer B.Cu) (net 4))
 (segment (start 144.78 107.95) (end 127.127 107.95) (width 0.635) (layer B.Cu) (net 4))
 (segment (start 126.9873 134.6327) (end 127 134.62) (width 0.635) (layer F.Cu) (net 5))
 (segment (start 128.143 124.523) (end 128.03 124.41) (width 0.635) (layer F.Cu) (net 5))
 (segment (start 128.03 126.125) (end 128.03 124.41) (width 0.635) (layer F.Cu) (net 5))
 (segment (start 129.54 127.635) (end 128.03 126.125) (width 0.635) (layer F.Cu) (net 5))
 (segment (start 131.0425 127.635) (end 129.54 127.635) (width 0.635) (layer F.Cu) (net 5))
 (segment (start 126.9873 135.15848) (end 126.9873 134.6327) (width 0.635) (layer F.Cu) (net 5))
 (segment (start 126.365 128.27) (end 128.03 126.605) (width 0.635) (layer F.Cu) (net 5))
 (segment (start 126.365 133.3754) (end 126.365 128.27) (width 0.635) (layer F.Cu) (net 5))
 (segment (start 126.9873 133.9977) (end 126.365 133.3754) (width 0.635) (layer F.Cu) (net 5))
 (segment (start 128.03 126.605) (end 128.03 126.125) (width 0.635) (layer F.Cu) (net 5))
 (segment (start 126.9873 135.15848) (end 126.9873 133.9977) (width 0.635) (layer F.Cu) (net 5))
 (segment (start 121.745 130.81) (end 121.745 127.81) (width 0.635) (layer F.Cu) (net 10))
 (segment (start 121.745 127.81) (end 121.745 127.81) (width 0.635) (layer F.Cu) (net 10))
 (segment (start 126.1325 110.49) (end 127.635 110.49) (width 0.635) (layer F.Cu) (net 10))
 (segment (start 127.635 110.49) (end 127.635 110.49) (width 0.635) (layer F.Cu) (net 10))
 (via (at 127.635 110.49) (size 0.8) (drill 0.4) (layers F.Cu B.Cu) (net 10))
 (segment (start 121.745 127.81) (end 121.745 127.81) (width 0.635) (layer F.Cu) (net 10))
 (via (at 121.745 127.81) (size 0.8) (drill 0.4) (layers F.Cu B.Cu) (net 10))
 (segment (start 129.54 120.015) (end 127.3175 122.2375) (width 0.635) (layer B.Cu) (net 10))
 (segment (start 129.54 111.125) (end 129.54 120.015) (width 0.635) (layer B.Cu) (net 10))
 (segment (start 128.905 110.49) (end 129.54 111.125) (width 0.635) (layer B.Cu) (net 10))
 (segment (start 127.635 110.49) (end 128.905 110.49) (width 0.635) (layer B.Cu) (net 10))
 (segment (start 127.3175 122.2375) (end 121.92 127.635) (width 0.635) (layer B.Cu) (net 10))
 (segment (start 127.635 121.92) (end 127.3175 122.2375) (width 0.635) (layer B.Cu) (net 10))
 (segment (start 144.535 131.095) (end 143.55 132.08) (width 0.635) (layer F.Cu) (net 14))
 (segment (start 144.535 124.19) (end 144.535 131.095) (width 0.635) (layer F.Cu) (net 14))
 (segment (start 137.906 130.15) (end 137.931 130.175) (width 0.635) (layer F.Cu) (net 13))
 (segment (start 137.906 127.635) (end 137.906 130.15) (width 0.635) (layer F.Cu) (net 13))
 (segment (start 135.645 124.19) (end 135.645 125.993) (width 0.635) (layer F.Cu) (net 12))
 (segment (start 135.906 126.254) (end 135.906 127.635) (width 0.635) (layer F.Cu) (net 12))
 (segment (start 135.645 125.993) (end 135.906 126.254) (width 0.635) (layer F.Cu) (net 12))
 (segment (start 133.828 131.602) (end 133.828 133.215) (width 0.4) (layer F.Cu) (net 6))
 (segment (start 133.828 131.602) (end 133.828 131.602) (width 0.254) (layer F.Cu) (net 6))
 (segment (start 128.4859 135.15848) (end 128.4859 134.4041) (width 0.4) (layer F.Cu) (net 6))
 (segment (start 128.4859 134.4041) (end 131.445 131.445) (width 0.4) (layer F.Cu) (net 6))
 (segment (start 133.671 131.445) (end 133.828 131.602) (width 0.4) (layer F.Cu) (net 6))
 (segment (start 131.445 131.445) (end 133.671 131.445) (width 0.4) (layer F.Cu) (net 6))
 (segment (start 151.86 110.49) (end 148.59 110.49) (width 0.635) (layer F.Cu) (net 2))
 (segment (start 152.4 109.95) (end 151.86 110.49) (width 0.635) (layer F.Cu) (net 2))
 (segment (start 151.67 111.76) (end 148.59 111.76) (width 0.635) (layer F.Cu) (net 3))
 (segment (start 152.4 112.49) (end 151.67 111.76) (width 0.635) (layer F.Cu) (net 3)))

